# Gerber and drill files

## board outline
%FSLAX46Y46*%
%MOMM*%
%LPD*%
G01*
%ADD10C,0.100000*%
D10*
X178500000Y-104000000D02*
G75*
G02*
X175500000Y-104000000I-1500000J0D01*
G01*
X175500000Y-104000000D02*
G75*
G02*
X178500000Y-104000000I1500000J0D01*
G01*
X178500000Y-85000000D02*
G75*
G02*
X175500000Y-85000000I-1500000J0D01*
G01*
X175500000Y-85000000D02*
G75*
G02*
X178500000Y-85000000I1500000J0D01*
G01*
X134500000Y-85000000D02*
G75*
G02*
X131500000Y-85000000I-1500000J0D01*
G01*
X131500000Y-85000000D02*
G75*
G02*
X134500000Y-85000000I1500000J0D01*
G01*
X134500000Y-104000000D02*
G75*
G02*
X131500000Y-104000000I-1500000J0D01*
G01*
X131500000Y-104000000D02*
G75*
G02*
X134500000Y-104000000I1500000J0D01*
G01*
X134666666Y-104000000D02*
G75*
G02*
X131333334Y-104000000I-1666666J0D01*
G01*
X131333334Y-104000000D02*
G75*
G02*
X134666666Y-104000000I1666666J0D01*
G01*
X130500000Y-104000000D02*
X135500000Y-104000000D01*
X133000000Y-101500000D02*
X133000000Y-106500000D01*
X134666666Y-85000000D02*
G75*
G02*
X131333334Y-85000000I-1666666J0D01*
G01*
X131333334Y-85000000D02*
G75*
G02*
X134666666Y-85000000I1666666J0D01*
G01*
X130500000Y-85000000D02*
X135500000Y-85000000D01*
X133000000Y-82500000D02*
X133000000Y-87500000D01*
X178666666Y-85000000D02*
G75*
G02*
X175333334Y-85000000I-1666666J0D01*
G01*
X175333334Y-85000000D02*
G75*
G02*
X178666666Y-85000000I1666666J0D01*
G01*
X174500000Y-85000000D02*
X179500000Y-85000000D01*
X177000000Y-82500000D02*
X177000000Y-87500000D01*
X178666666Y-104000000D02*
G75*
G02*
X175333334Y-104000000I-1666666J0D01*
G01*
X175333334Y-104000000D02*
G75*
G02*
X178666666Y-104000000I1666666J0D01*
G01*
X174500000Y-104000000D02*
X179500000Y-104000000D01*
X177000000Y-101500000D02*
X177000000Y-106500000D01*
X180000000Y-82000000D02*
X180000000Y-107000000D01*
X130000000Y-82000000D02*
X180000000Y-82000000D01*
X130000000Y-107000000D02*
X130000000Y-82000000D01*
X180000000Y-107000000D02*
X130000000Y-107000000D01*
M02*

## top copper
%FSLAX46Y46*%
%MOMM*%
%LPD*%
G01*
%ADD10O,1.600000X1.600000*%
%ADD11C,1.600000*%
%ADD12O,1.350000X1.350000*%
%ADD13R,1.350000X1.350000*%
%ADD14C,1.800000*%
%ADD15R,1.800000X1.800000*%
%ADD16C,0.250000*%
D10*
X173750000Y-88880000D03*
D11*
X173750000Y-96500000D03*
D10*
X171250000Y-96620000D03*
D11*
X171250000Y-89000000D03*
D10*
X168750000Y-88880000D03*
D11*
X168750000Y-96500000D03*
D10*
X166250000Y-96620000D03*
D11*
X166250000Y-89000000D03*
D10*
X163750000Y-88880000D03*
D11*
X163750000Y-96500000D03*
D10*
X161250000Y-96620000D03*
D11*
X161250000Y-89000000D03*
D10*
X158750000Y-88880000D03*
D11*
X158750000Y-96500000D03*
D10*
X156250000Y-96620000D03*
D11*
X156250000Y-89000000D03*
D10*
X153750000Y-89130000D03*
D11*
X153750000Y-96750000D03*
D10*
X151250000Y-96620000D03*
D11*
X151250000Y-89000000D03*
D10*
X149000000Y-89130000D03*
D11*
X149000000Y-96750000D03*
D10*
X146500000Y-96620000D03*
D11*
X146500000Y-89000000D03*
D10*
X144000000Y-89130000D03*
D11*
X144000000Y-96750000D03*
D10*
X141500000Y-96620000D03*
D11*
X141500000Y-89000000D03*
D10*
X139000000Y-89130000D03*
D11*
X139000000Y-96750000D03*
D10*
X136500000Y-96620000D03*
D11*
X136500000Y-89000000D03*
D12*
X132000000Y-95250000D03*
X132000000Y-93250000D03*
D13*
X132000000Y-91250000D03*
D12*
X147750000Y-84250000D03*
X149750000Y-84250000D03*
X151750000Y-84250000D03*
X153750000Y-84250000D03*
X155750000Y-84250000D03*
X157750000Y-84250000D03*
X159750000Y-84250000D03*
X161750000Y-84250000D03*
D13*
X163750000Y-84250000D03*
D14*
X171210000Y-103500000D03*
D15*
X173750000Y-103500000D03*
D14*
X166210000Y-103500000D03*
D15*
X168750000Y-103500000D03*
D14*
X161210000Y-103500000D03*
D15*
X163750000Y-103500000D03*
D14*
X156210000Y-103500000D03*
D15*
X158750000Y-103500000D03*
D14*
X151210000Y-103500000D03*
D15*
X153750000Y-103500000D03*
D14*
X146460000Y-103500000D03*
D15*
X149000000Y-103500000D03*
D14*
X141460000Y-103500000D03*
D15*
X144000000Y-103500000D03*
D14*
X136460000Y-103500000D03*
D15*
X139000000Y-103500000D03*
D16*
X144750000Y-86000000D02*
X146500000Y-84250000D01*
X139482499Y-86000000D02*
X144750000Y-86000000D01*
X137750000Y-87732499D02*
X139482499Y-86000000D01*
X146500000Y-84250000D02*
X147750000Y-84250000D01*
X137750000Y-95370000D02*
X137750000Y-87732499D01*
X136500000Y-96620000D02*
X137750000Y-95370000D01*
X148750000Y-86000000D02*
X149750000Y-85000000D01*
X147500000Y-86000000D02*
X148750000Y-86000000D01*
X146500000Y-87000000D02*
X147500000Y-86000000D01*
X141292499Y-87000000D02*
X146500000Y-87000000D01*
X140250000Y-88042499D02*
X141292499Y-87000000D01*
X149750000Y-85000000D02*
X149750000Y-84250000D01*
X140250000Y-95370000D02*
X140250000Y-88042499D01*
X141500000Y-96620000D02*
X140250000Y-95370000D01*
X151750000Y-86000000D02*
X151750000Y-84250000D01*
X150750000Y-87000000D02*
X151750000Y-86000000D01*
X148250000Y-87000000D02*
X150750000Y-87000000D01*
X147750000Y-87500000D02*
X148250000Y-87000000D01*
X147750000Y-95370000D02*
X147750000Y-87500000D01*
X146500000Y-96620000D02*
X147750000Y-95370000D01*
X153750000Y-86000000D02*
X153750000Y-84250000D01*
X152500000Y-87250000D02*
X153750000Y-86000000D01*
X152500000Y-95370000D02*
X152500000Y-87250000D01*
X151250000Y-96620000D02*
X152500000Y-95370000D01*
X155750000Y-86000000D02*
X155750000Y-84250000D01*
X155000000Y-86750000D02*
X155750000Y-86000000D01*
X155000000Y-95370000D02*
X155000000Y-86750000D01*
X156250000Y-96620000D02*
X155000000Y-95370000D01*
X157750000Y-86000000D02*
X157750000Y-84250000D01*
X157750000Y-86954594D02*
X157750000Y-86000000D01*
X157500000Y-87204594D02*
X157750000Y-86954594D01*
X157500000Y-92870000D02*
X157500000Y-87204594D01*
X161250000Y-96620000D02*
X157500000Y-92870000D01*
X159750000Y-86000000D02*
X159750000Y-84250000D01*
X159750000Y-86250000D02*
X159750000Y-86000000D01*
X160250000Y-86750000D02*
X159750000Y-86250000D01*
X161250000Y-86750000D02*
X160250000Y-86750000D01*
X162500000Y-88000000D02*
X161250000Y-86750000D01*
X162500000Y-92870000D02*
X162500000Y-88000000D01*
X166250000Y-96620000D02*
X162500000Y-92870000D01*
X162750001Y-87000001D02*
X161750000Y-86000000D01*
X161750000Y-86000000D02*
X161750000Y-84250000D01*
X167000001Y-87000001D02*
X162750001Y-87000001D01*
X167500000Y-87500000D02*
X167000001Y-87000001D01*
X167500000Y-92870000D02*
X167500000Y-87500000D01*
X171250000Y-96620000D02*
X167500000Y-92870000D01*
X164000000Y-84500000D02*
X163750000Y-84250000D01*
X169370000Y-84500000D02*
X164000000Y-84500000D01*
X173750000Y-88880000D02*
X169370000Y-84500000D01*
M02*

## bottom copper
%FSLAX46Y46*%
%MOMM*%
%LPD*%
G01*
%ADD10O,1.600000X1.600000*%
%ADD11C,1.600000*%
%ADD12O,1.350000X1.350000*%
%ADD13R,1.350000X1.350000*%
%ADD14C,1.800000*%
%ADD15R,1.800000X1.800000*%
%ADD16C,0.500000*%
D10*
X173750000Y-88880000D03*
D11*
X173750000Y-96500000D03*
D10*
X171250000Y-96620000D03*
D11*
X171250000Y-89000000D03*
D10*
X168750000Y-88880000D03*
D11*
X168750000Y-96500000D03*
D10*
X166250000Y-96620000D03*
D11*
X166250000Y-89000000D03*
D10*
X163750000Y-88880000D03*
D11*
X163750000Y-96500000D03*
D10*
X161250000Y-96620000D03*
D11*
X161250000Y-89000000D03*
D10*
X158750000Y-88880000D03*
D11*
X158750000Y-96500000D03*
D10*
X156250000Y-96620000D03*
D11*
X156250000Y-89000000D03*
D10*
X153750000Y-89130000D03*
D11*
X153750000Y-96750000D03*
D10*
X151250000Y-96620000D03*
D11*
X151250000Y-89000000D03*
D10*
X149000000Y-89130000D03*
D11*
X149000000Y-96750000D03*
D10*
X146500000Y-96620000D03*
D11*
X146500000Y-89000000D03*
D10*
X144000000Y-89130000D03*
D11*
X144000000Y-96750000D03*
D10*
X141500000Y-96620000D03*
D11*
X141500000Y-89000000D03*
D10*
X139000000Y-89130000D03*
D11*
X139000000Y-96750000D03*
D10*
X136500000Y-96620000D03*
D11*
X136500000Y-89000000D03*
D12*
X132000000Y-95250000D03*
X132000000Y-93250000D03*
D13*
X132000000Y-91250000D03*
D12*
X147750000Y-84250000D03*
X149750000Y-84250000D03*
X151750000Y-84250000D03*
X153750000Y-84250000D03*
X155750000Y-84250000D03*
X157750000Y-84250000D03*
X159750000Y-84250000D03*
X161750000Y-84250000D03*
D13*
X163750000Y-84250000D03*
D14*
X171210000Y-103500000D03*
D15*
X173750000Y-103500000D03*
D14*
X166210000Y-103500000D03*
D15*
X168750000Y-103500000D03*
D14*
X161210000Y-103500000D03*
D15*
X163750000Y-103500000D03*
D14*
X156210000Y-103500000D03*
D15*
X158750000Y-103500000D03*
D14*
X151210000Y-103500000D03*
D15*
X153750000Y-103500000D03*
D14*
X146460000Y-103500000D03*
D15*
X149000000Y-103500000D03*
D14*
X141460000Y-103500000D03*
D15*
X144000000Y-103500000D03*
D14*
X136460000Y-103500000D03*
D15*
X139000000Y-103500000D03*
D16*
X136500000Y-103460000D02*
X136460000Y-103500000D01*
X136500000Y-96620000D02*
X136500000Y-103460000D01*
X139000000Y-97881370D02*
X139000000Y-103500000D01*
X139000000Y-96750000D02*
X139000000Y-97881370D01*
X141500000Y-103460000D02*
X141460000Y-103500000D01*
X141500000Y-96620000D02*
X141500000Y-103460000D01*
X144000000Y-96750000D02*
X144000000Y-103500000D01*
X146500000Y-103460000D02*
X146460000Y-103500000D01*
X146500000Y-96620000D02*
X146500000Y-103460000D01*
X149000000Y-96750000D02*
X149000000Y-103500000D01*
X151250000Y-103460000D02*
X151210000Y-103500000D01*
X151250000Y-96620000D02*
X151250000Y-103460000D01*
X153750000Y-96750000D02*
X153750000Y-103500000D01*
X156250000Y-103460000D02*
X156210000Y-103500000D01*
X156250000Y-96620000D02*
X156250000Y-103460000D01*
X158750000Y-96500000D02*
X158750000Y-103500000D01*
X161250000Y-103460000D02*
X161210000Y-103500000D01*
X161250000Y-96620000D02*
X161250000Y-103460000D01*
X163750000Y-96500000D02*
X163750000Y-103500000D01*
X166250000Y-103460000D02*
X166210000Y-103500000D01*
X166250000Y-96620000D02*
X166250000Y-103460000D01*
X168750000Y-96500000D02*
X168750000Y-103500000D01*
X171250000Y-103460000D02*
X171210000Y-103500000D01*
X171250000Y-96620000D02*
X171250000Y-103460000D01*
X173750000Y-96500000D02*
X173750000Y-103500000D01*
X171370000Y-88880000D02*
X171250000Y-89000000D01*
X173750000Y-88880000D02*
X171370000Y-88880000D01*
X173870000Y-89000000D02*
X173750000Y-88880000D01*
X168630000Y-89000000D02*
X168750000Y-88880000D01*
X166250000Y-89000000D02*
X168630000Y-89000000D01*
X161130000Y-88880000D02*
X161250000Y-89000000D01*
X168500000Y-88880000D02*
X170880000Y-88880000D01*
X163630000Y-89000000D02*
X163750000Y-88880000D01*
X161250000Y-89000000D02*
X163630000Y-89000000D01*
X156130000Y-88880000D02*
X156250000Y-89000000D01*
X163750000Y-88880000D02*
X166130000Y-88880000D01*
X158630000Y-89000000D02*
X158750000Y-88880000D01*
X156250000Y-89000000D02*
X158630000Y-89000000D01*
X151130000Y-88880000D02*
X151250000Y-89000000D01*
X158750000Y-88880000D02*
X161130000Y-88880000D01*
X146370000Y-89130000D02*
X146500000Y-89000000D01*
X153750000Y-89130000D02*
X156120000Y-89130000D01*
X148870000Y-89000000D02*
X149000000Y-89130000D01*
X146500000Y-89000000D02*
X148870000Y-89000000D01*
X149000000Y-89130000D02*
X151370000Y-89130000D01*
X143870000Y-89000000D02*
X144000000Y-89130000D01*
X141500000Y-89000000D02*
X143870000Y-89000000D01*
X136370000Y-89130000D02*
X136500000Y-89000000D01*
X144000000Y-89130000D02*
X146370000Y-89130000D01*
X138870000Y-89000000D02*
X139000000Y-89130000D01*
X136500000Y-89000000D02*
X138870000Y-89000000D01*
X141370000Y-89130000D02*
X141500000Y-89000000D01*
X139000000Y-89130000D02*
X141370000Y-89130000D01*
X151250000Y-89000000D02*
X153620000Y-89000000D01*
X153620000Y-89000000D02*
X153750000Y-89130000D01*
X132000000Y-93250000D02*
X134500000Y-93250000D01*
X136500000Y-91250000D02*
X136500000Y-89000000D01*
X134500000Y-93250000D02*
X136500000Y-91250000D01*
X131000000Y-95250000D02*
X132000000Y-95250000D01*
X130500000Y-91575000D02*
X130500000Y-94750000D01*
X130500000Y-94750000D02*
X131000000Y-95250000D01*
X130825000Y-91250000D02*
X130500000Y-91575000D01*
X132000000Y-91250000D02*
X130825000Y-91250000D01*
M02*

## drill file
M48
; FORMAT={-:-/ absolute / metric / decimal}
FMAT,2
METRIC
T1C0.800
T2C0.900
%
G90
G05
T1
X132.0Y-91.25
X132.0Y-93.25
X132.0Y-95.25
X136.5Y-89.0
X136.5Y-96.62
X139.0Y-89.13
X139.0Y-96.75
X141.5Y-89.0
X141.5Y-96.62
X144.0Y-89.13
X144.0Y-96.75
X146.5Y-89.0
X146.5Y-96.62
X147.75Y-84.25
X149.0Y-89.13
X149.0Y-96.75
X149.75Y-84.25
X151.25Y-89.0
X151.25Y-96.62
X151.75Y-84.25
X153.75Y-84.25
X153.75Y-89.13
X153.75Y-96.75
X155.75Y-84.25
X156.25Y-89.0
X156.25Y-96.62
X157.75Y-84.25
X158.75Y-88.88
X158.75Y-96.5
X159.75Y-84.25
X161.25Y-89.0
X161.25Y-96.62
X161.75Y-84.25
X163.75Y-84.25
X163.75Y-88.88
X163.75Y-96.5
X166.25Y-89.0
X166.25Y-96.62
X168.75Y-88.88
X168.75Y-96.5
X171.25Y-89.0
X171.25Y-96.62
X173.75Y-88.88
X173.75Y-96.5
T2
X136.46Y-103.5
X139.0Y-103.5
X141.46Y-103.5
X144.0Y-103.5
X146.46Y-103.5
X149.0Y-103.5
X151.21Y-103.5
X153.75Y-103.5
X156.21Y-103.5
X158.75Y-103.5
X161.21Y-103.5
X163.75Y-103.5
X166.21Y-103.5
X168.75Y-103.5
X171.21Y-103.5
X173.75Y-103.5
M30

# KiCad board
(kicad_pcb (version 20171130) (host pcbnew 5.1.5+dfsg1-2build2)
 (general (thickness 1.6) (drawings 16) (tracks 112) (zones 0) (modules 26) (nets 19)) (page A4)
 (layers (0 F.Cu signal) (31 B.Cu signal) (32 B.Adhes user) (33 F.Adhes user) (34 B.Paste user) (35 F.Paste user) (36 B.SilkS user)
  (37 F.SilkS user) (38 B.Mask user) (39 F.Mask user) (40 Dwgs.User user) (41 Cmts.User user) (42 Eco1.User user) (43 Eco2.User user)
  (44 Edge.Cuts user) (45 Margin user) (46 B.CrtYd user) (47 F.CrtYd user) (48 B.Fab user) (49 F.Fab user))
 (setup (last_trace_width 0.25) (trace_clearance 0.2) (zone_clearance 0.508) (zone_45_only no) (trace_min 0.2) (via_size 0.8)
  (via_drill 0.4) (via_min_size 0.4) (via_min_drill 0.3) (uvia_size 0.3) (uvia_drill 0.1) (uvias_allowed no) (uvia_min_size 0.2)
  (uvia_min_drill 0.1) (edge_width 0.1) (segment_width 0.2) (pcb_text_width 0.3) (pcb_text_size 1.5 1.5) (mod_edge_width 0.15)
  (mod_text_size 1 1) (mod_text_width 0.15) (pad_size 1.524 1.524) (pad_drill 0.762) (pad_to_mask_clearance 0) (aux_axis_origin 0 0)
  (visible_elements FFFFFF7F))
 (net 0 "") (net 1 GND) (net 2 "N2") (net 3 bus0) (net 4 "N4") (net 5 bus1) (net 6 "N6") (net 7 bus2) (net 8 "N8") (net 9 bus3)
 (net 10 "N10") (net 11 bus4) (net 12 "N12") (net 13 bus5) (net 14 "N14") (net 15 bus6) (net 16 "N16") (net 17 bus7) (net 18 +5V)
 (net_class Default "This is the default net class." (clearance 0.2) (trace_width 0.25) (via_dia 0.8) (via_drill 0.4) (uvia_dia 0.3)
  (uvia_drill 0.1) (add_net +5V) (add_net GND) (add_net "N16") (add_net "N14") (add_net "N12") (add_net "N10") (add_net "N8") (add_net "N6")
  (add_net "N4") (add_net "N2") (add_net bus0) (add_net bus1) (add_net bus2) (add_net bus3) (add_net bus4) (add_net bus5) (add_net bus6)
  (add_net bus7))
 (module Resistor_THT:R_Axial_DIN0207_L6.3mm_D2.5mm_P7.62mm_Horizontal (layer F.Cu) (at 173.75 96.5 90)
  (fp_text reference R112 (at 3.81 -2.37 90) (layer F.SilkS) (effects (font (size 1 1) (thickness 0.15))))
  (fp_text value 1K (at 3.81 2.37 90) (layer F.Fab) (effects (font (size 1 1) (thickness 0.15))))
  (pad 2 thru_hole oval (at 7.62 0 90) (size 1.6 1.6) (drill 0.8) (layers *.Cu *.Mask) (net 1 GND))
  (pad 1 thru_hole circle (at 0 0 90) (size 1.6 1.6) (drill 0.8) (layers *.Cu *.Mask) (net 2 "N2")))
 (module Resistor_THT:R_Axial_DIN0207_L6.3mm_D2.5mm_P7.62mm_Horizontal (layer F.Cu) (at 171.25 89 270)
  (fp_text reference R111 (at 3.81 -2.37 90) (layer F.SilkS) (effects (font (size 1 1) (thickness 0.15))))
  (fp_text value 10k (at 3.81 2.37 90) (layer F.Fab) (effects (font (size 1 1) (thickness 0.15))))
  (pad 2 thru_hole oval (at 7.62 0 270) (size 1.6 1.6) (drill 0.8) (layers *.Cu *.Mask) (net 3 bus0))
  (pad 1 thru_hole circle (at 0 0 270) (size 1.6 1.6) (drill 0.8) (layers *.Cu *.Mask) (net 1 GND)))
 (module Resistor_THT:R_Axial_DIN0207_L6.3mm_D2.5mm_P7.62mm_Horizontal (layer F.Cu) (at 168.75 96.5 90)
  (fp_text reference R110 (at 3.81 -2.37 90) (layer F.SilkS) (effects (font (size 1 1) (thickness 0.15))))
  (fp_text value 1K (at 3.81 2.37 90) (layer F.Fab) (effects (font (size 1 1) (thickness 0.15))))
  (pad 2 thru_hole oval (at 7.62 0 90) (size 1.6 1.6) (drill 0.8) (layers *.Cu *.Mask) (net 1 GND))
  (pad 1 thru_hole circle (at 0 0 90) (size 1.6 1.6) (drill 0.8) (layers *.Cu *.Mask) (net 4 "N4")))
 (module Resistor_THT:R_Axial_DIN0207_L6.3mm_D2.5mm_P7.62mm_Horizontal (layer F.Cu) (at 166.25 89 270)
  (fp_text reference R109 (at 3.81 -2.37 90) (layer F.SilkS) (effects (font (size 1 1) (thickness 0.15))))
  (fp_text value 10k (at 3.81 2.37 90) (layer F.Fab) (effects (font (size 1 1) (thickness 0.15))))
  (pad 2 thru_hole oval (at 7.62 0 270) (size 1.6 1.6) (drill 0.8) (layers *.Cu *.Mask) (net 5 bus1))
  (pad 1 thru_hole circle (at 0 0 270) (size 1.6 1.6) (drill 0.8) (layers *.Cu *.Mask) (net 1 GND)))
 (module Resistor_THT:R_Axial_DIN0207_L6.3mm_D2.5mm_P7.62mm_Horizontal (layer F.Cu) (at 163.75 96.5 90)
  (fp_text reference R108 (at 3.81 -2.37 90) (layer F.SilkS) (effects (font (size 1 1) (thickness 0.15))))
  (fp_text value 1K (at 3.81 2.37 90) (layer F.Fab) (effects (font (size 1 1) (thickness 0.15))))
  (pad 2 thru_hole oval (at 7.62 0 90) (size 1.6 1.6) (drill 0.8) (layers *.Cu *.Mask) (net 1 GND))
  (pad 1 thru_hole circle (at 0 0 90) (size 1.6 1.6) (drill 0.8) (layers *.Cu *.Mask) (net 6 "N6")))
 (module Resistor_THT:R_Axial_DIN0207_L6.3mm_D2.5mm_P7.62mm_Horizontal (layer F.Cu) (at 161.25 89 270)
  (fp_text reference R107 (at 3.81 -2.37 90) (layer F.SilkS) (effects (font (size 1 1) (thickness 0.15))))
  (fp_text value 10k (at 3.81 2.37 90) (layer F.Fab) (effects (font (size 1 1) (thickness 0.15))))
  (pad 2 thru_hole oval (at 7.62 0 270) (size 1.6 1.6) (drill 0.8) (layers *.Cu *.Mask) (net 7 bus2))
  (pad 1 thru_hole circle (at 0 0 270) (size 1.6 1.6) (drill 0.8) (layers *.Cu *.Mask) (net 1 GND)))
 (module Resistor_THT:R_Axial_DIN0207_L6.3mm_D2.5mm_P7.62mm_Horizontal (layer F.Cu) (at 158.75 96.5 90)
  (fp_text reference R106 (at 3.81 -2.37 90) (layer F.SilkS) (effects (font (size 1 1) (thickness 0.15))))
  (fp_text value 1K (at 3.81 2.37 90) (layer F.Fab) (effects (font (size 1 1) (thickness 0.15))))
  (pad 2 thru_hole oval (at 7.62 0 90) (size 1.6 1.6) (drill 0.8) (layers *.Cu *.Mask) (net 1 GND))
  (pad 1 thru_hole circle (at 0 0 90) (size 1.6 1.6) (drill 0.8) (layers *.Cu *.Mask) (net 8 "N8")))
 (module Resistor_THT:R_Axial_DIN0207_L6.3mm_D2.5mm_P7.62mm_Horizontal (layer F.Cu) (at 156.25 89 270)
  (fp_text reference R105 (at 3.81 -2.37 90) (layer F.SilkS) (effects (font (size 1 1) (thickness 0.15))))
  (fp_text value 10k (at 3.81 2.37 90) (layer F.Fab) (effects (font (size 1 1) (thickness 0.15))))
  (pad 2 thru_hole oval (at 7.62 0 270) (size 1.6 1.6) (drill 0.8) (layers *.Cu *.Mask) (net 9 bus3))
  (pad 1 thru_hole circle (at 0 0 270) (size 1.6 1.6) (drill 0.8) (layers *.Cu *.Mask) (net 1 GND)))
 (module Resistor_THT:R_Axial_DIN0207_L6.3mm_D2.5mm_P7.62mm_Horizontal (layer F.Cu) (at 153.75 96.75 90)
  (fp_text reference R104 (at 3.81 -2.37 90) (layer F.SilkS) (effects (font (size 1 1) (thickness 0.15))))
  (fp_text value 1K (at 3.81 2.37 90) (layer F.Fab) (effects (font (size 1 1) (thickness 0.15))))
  (pad 2 thru_hole oval (at 7.62 0 90) (size 1.6 1.6) (drill 0.8) (layers *.Cu *.Mask) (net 1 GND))
  (pad 1 thru_hole circle (at 0 0 90) (size 1.6 1.6) (drill 0.8) (layers *.Cu *.Mask) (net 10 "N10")))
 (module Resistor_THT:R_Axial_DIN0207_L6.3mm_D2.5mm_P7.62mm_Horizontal (layer F.Cu) (at 151.25 89 270)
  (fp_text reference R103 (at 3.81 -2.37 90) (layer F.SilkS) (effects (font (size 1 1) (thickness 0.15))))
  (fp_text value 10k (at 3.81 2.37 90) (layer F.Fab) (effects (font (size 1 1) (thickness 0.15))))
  (pad 2 thru_hole oval (at 7.62 0 270) (size 1.6 1.6) (drill 0.8) (layers *.Cu *.Mask) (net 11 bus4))
  (pad 1 thru_hole circle (at 0 0 270) (size 1.6 1.6) (drill 0.8) (layers *.Cu *.Mask) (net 1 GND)))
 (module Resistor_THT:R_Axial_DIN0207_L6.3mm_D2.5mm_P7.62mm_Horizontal (layer F.Cu) (at 149 96.75 90)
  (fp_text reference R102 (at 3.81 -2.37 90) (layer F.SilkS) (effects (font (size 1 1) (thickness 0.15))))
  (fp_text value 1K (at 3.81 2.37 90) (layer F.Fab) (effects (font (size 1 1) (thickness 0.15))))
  (pad 2 thru_hole oval (at 7.62 0 90) (size 1.6 1.6) (drill 0.8) (layers *.Cu *.Mask) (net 1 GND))
  (pad 1 thru_hole circle (at 0 0 90) (size 1.6 1.6) (drill 0.8) (layers *.Cu *.Mask) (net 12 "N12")))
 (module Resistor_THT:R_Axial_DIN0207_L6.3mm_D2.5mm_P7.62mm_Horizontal (layer F.Cu) (at 146.5 89 270)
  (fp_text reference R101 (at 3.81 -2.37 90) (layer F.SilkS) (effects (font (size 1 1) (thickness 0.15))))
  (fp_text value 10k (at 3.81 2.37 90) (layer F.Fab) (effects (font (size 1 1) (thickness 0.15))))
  (pad 2 thru_hole oval (at 7.62 0 270) (size 1.6 1.6) (drill 0.8) (layers *.Cu *.Mask) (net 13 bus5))
  (pad 1 thru_hole circle (at 0 0 270) (size 1.6 1.6) (drill 0.8) (layers *.Cu *.Mask) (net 1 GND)))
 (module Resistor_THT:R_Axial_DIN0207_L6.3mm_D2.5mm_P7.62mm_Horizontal (layer F.Cu) (at 144 96.75 90)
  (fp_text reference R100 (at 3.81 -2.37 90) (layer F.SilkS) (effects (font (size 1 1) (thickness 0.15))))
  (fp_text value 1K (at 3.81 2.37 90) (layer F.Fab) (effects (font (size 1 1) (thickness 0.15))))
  (pad 2 thru_hole oval (at 7.62 0 90) (size 1.6 1.6) (drill 0.8) (layers *.Cu *.Mask) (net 1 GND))
  (pad 1 thru_hole circle (at 0 0 90) (size 1.6 1.6) (drill 0.8) (layers *.Cu *.Mask) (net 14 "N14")))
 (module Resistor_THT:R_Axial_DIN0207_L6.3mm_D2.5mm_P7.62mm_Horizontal (layer F.Cu) (at 141.5 89 270)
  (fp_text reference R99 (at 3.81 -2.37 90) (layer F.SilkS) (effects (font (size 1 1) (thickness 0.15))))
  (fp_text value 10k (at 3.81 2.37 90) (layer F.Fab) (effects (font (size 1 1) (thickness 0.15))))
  (pad 2 thru_hole oval (at 7.62 0 270) (size 1.6 1.6) (drill 0.8) (layers *.Cu *.Mask) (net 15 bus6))
  (pad 1 thru_hole circle (at 0 0 270) (size 1.6 1.6) (drill 0.8) (layers *.Cu *.Mask) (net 1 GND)))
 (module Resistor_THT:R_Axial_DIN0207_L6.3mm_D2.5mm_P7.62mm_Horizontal (layer F.Cu) (at 139 96.75 90)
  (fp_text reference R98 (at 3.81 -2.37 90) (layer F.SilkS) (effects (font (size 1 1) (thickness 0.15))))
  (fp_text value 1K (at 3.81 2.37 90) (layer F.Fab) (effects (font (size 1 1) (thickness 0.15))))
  (pad 2 thru_hole oval (at 7.62 0 90) (size 1.6 1.6) (drill 0.8) (layers *.Cu *.Mask) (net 1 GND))
  (pad 1 thru_hole circle (at 0 0 90) (size 1.6 1.6) (drill 0.8) (layers *.Cu *.Mask) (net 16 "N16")))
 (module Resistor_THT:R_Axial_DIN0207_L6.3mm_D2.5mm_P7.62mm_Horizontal (layer F.Cu) (at 136.5 89 270)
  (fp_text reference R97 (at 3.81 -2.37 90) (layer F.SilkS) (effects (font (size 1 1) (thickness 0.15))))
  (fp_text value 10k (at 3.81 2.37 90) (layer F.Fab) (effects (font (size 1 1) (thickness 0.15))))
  (pad 2 thru_hole oval (at 7.62 0 270) (size 1.6 1.6) (drill 0.8) (layers *.Cu *.Mask) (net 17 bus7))
  (pad 1 thru_hole circle (at 0 0 270) (size 1.6 1.6) (drill 0.8) (layers *.Cu *.Mask) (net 1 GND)))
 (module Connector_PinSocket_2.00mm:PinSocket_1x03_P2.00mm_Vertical (layer F.Cu) (at 132 91.25)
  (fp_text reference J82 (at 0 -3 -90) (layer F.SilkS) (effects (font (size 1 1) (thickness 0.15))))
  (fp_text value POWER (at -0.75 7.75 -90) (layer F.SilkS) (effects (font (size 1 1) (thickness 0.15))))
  (pad 3 thru_hole oval (at 0 4) (size 1.35 1.35) (drill 0.8) (layers *.Cu *.Mask) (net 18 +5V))
  (pad 2 thru_hole oval (at 0 2) (size 1.35 1.35) (drill 0.8) (layers *.Cu *.Mask) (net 1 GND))
  (pad 1 thru_hole rect (at 0 0) (size 1.35 1.35) (drill 0.8) (layers *.Cu *.Mask) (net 18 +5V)))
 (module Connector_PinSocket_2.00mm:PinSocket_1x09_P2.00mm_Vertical (layer F.Cu) (at 163.75 84.25 270)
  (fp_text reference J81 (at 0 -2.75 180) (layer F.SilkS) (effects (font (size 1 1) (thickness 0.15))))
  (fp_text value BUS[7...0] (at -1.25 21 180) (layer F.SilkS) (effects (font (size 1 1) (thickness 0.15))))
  (pad 9 thru_hole oval (at 0 16 270) (size 1.35 1.35) (drill 0.8) (layers *.Cu *.Mask) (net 17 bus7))
  (pad 8 thru_hole oval (at 0 14 270) (size 1.35 1.35) (drill 0.8) (layers *.Cu *.Mask) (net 15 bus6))
  (pad 7 thru_hole oval (at 0 12 270) (size 1.35 1.35) (drill 0.8) (layers *.Cu *.Mask) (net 13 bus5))
  (pad 6 thru_hole oval (at 0 10 270) (size 1.35 1.35) (drill 0.8) (layers *.Cu *.Mask) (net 11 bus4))
  (pad 5 thru_hole oval (at 0 8 270) (size 1.35 1.35) (drill 0.8) (layers *.Cu *.Mask) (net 9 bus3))
  (pad 4 thru_hole oval (at 0 6 270) (size 1.35 1.35) (drill 0.8) (layers *.Cu *.Mask) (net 7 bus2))
  (pad 3 thru_hole oval (at 0 4 270) (size 1.35 1.35) (drill 0.8) (layers *.Cu *.Mask) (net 5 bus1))
  (pad 2 thru_hole oval (at 0 2 270) (size 1.35 1.35) (drill 0.8) (layers *.Cu *.Mask) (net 3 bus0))
  (pad 1 thru_hole rect (at 0 0 270) (size 1.35 1.35) (drill 0.8) (layers *.Cu *.Mask) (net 1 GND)))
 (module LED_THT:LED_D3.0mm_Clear (layer F.Cu) (at 173.75 103.5 180)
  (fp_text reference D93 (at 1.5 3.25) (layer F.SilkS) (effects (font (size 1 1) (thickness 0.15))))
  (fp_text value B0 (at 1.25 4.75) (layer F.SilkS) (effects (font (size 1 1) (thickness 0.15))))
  (pad 2 thru_hole circle (at 2.54 0 180) (size 1.8 1.8) (drill 0.9) (layers *.Cu *.Mask) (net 3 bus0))
  (pad 1 thru_hole rect (at 0 0 180) (size 1.8 1.8) (drill 0.9) (layers *.Cu *.Mask) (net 2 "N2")))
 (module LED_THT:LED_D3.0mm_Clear (layer F.Cu) (at 168.75 103.5 180)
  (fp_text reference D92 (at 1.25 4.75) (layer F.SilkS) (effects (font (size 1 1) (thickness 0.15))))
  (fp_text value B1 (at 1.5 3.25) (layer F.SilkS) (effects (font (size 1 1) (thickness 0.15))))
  (pad 2 thru_hole circle (at 2.54 0 180) (size 1.8 1.8) (drill 0.9) (layers *.Cu *.Mask) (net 5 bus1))
  (pad 1 thru_hole rect (at 0 0 180) (size 1.8 1.8) (drill 0.9) (layers *.Cu *.Mask) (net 4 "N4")))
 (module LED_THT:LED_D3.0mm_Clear (layer F.Cu) (at 163.75 103.5 180)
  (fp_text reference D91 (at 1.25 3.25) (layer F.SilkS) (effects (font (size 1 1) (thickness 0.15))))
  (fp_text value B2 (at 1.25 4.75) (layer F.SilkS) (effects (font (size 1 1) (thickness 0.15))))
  (pad 2 thru_hole circle (at 2.54 0 180) (size 1.8 1.8) (drill 0.9) (layers *.Cu *.Mask) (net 7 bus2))
  (pad 1 thru_hole rect (at 0 0 180) (size 1.8 1.8) (drill 0.9) (layers *.Cu *.Mask) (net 6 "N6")))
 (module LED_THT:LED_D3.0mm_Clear (layer F.Cu) (at 158.75 103.5 180)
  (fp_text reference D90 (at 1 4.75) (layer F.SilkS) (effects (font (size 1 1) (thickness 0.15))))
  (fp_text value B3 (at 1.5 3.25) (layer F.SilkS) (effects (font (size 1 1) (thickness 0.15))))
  (pad 2 thru_hole circle (at 2.54 0 180) (size 1.8 1.8) (drill 0.9) (layers *.Cu *.Mask) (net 9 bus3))
  (pad 1 thru_hole rect (at 0 0 180) (size 1.8 1.8) (drill 0.9) (layers *.Cu *.Mask) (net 8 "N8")))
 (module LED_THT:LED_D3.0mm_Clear (layer F.Cu) (at 153.75 103.5 180)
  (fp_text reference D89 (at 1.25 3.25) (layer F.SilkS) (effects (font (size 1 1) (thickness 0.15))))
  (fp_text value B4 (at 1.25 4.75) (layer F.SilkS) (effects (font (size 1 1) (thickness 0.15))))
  (pad 2 thru_hole circle (at 2.54 0 180) (size 1.8 1.8) (drill 0.9) (layers *.Cu *.Mask) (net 11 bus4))
  (pad 1 thru_hole rect (at 0 0 180) (size 1.8 1.8) (drill 0.9) (layers *.Cu *.Mask) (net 10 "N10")))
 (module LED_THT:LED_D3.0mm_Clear (layer F.Cu) (at 149 103.5 180)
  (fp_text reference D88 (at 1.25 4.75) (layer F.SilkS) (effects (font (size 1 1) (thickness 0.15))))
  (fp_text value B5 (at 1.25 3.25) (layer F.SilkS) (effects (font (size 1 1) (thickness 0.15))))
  (pad 2 thru_hole circle (at 2.54 0 180) (size 1.8 1.8) (drill 0.9) (layers *.Cu *.Mask) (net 13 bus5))
  (pad 1 thru_hole rect (at 0 0 180) (size 1.8 1.8) (drill 0.9) (layers *.Cu *.Mask) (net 12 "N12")))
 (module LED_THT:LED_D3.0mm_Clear (layer F.Cu) (at 144 103.5 180)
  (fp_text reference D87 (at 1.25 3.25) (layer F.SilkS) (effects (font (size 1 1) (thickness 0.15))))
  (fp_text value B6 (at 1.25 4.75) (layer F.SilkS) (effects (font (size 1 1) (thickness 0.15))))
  (pad 2 thru_hole circle (at 2.54 0 180) (size 1.8 1.8) (drill 0.9) (layers *.Cu *.Mask) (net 15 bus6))
  (pad 1 thru_hole rect (at 0 0 180) (size 1.8 1.8) (drill 0.9) (layers *.Cu *.Mask) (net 14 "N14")))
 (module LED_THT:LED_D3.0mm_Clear (layer F.Cu) (at 139 103.5 180)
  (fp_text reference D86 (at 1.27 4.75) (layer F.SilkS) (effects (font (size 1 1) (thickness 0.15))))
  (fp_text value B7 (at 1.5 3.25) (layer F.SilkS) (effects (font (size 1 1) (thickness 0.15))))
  (pad 2 thru_hole circle (at 2.54 0 180) (size 1.8 1.8) (drill 0.9) (layers *.Cu *.Mask) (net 17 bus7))
  (pad 1 thru_hole rect (at 0 0 180) (size 1.8 1.8) (drill 0.9) (layers *.Cu *.Mask) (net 16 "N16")))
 (gr_circle (center 177 104) (end 178.5 104) (layer Edge.Cuts) (width 0.1))
 (gr_circle (center 177 85) (end 178.5 85) (layer Edge.Cuts) (width 0.1))
 (gr_circle (center 133 85) (end 134.5 85) (layer Edge.Cuts) (width 0.1))
 (gr_circle (center 133 104) (end 134.5 104) (layer Edge.Cuts) (width 0.1))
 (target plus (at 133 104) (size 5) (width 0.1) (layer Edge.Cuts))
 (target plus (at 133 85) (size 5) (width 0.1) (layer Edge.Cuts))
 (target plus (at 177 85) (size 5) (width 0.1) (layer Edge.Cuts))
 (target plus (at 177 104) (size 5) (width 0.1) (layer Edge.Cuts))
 (gr_line (start 180 82) (end 180 107) (layer Edge.Cuts) (width 0.1))
 (gr_line (start 130 82) (end 180 82) (layer Edge.Cuts) (width 0.1))
 (gr_line (start 130 107) (end 130 82) (layer Edge.Cuts) (width 0.1))
 (gr_line (start 180 107) (end 130 107) (layer Edge.Cuts) (width 0.1))
 (segment (start 136.5 103.46) (end 136.46 103.5) (width 0.5) (layer B.Cu) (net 17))
 (segment (start 136.5 96.62) (end 136.5 103.46) (width 0.5) (layer B.Cu) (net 17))
 (segment (start 144.75 86) (end 146.5 84.25) (width 0.25) (layer F.Cu) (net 17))
 (segment (start 139.482499 86) (end 144.75 86) (width 0.25) (layer F.Cu) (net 17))
 (segment (start 137.75 87.732499) (end 139.482499 86) (width 0.25) (layer F.Cu) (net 17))
 (segment (start 146.5 84.25) (end 147.75 84.25) (width 0.25) (layer F.Cu) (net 17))
 (segment (start 137.75 95.37) (end 137.75 87.732499) (width 0.25) (layer F.Cu) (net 17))
 (segment (start 136.5 96.62) (end 137.75 95.37) (width 0.25) (layer F.Cu) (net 17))
 (segment (start 139 97.88137) (end 139 103.5) (width 0.5) (layer B.Cu) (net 16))
 (segment (start 139 96.75) (end 139 97.88137) (width 0.5) (layer B.Cu) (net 16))
 (segment (start 141.5 103.46) (end 141.46 103.5) (width 0.5) (layer B.Cu) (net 15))
 (segment (start 141.5 96.62) (end 141.5 103.46) (width 0.5) (layer B.Cu) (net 15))
 (segment (start 148.75 86) (end 149.75 85) (width 0.25) (layer F.Cu) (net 15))
 (segment (start 147.5 86) (end 148.75 86) (width 0.25) (layer F.Cu) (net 15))
 (segment (start 146.5 87) (end 147.5 86) (width 0.25) (layer F.Cu) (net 15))
 (segment (start 141.292499 87) (end 146.5 87) (width 0.25) (layer F.Cu) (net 15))
 (segment (start 140.25 88.042499) (end 141.292499 87) (width 0.25) (layer F.Cu) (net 15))
 (segment (start 149.75 85) (end 149.75 84.25) (width 0.25) (layer F.Cu) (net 15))
 (segment (start 140.25 95.37) (end 140.25 88.042499) (width 0.25) (layer F.Cu) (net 15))
 (segment (start 141.5 96.62) (end 140.25 95.37) (width 0.25) (layer F.Cu) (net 15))
 (segment (start 144 96.75) (end 144 103.5) (width 0.5) (layer B.Cu) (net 14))
 (segment (start 146.5 103.46) (end 146.46 103.5) (width 0.5) (layer B.Cu) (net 13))
 (segment (start 146.5 96.62) (end 146.5 103.46) (width 0.5) (layer B.Cu) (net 13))
 (segment (start 151.75 86) (end 151.75 84.25) (width 0.25) (layer F.Cu) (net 13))
 (segment (start 150.75 87) (end 151.75 86) (width 0.25) (layer F.Cu) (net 13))
 (segment (start 148.25 87) (end 150.75 87) (width 0.25) (layer F.Cu) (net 13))
 (segment (start 147.75 87.5) (end 148.25 87) (width 0.25) (layer F.Cu) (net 13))
 (segment (start 147.75 95.37) (end 147.75 87.5) (width 0.25) (layer F.Cu) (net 13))
 (segment (start 146.5 96.62) (end 147.75 95.37) (width 0.25) (layer F.Cu) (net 13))
 (segment (start 149 96.75) (end 149 103.5) (width 0.5) (layer B.Cu) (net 12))
 (segment (start 151.25 103.46) (end 151.21 103.5) (width 0.5) (layer B.Cu) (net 11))
 (segment (start 151.25 96.62) (end 151.25 103.46) (width 0.5) (layer B.Cu) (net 11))
 (segment (start 153.75 86) (end 153.75 84.25) (width 0.25) (layer F.Cu) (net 11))
 (segment (start 152.5 87.25) (end 153.75 86) (width 0.25) (layer F.Cu) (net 11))
 (segment (start 152.5 95.37) (end 152.5 87.25) (width 0.25) (layer F.Cu) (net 11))
 (segment (start 151.25 96.62) (end 152.5 95.37) (width 0.25) (layer F.Cu) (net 11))
 (segment (start 153.75 96.75) (end 153.75 103.5) (width 0.5) (layer B.Cu) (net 10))
 (segment (start 156.25 103.46) (end 156.21 103.5) (width 0.5) (layer B.Cu) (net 9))
 (segment (start 156.25 96.62) (end 156.25 103.46) (width 0.5) (layer B.Cu) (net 9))
 (segment (start 155.75 86) (end 155.75 84.25) (width 0.25) (layer F.Cu) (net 9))
 (segment (start 155 86.75) (end 155.75 86) (width 0.25) (layer F.Cu) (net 9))
 (segment (start 155 95.37) (end 155 86.75) (width 0.25) (layer F.Cu) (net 9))
 (segment (start 156.25 96.62) (end 155 95.37) (width 0.25) (layer F.Cu) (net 9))
 (segment (start 158.75 96.5) (end 158.75 103.5) (width 0.5) (layer B.Cu) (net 8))
 (segment (start 161.25 103.46) (end 161.21 103.5) (width 0.5) (layer B.Cu) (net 7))
 (segment (start 161.25 96.62) (end 161.25 103.46) (width 0.5) (layer B.Cu) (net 7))
 (segment (start 157.75 86) (end 157.75 84.25) (width 0.25) (layer F.Cu) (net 7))
 (segment (start 157.75 86.954594) (end 157.75 86) (width 0.25) (layer F.Cu) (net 7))
 (segment (start 157.5 87.204594) (end 157.75 86.954594) (width 0.25) (layer F.Cu) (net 7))
 (segment (start 157.5 92.87) (end 157.5 87.204594) (width 0.25) (layer F.Cu) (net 7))
 (segment (start 161.25 96.62) (end 157.5 92.87) (width 0.25) (layer F.Cu) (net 7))
 (segment (start 163.75 96.5) (end 163.75 103.5) (width 0.5) (layer B.Cu) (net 6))
 (segment (start 166.25 103.46) (end 166.21 103.5) (width 0.5) (layer B.Cu) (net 5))
 (segment (start 166.25 96.62) (end 166.25 103.46) (width 0.5) (layer B.Cu) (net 5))
 (segment (start 159.75 86) (end 159.75 84.25) (width 0.25) (layer F.Cu) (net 5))
 (segment (start 159.75 86.25) (end 159.75 86) (width 0.25) (layer F.Cu) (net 5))
 (segment (start 160.25 86.75) (end 159.75 86.25) (width 0.25) (layer F.Cu) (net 5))
 (segment (start 161.25 86.75) (end 160.25 86.75) (width 0.25) (layer F.Cu) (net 5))
 (segment (start 162.5 88) (end 161.25 86.75) (width 0.25) (layer F.Cu) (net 5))
 (segment (start 162.5 92.87) (end 162.5 88) (width 0.25) (layer F.Cu) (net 5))
 (segment (start 166.25 96.62) (end 162.5 92.87) (width 0.25) (layer F.Cu) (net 5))
 (segment (start 168.75 96.5) (end 168.75 103.5) (width 0.5) (layer B.Cu) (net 4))
 (segment (start 171.25 103.46) (end 171.21 103.5) (width 0.5) (layer B.Cu) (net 3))
 (segment (start 171.25 96.62) (end 171.25 103.46) (width 0.5) (layer B.Cu) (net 3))
 (segment (start 162.750001 87.000001) (end 161.75 86) (width 0.25) (layer F.Cu) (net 3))
 (segment (start 161.75 86) (end 161.75 84.25) (width 0.25) (layer F.Cu) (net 3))
 (segment (start 167.000001 87.000001) (end 162.750001 87.000001) (width 0.25) (layer F.Cu) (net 3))
 (segment (start 167.5 87.5) (end 167.000001 87.000001) (width 0.25) (layer F.Cu) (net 3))
 (segment (start 167.5 92.87) (end 167.5 87.5) (width 0.25) (layer F.Cu) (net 3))
 (segment (start 171.25 96.62) (end 167.5 92.87) (width 0.25) (layer F.Cu) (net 3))
 (segment (start 173.75 96.5) (end 173.75 103.5) (width 0.5) (layer B.Cu) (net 2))
 (segment (start 171.37 88.88) (end 171.25 89) (width 0.5) (layer B.Cu) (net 1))
 (segment (start 173.75 88.88) (end 171.37 88.88) (width 0.5) (layer B.Cu) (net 1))
 (segment (start 173.87 89) (end 173.75 88.88) (width 0.5) (layer B.Cu) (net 1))
 (segment (start 168.63 89) (end 168.75 88.88) (width 0.5) (layer B.Cu) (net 1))
 (segment (start 166.25 89) (end 168.63 89) (width 0.5) (layer B.Cu) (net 1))
 (segment (start 161.13 88.88) (end 161.25 89) (width 0.5) (layer B.Cu) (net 1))
 (segment (start 168.5 88.88) (end 170.88 88.88) (width 0.5) (layer B.Cu) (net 1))
 (segment (start 163.63 89) (end 163.75 88.88) (width 0.5) (layer B.Cu) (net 1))
 (segment (start 161.25 89) (end 163.63 89) (width 0.5) (layer B.Cu) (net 1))
 (segment (start 156.13 88.88) (end 156.25 89) (width 0.5) (layer B.Cu) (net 1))
 (segment (start 163.75 88.88) (end 166.13 88.88) (width 0.5) (layer B.Cu) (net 1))
 (segment (start 158.63 89) (end 158.75 88.88) (width 0.5) (layer B.Cu) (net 1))
 (segment (start 156.25 89) (end 158.63 89) (width 0.5) (layer B.Cu) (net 1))
 (segment (start 151.13 88.88) (end 151.25 89) (width 0.5) (layer B.Cu) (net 1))
 (segment (start 158.75 88.88) (end 161.13 88.88) (width 0.5) (layer B.Cu) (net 1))
 (segment (start 146.37 89.13) (end 146.5 89) (width 0.5) (layer B.Cu) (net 1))
 (segment (start 153.75 89.13) (end 156.12 89.13) (width 0.5) (layer B.Cu) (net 1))
 (segment (start 148.87 89) (end 149 89.13) (width 0.5) (layer B.Cu) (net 1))
 (segment (start 146.5 89) (end 148.87 89) (width 0.5) (layer B.Cu) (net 1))
 (segment (start 149 89.13) (end 151.37 89.13) (width 0.5) (layer B.Cu) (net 1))
 (segment (start 143.87 89) (end 144 89.13) (width 0.5) (layer B.Cu) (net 1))
 (segment (start 141.5 89) (end 143.87 89) (width 0.5) (layer B.Cu) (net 1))
 (segment (start 136.37 89.13) (end 136.5 89) (width 0.5) (layer B.Cu) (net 1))
 (segment (start 144 89.13) (end 146.37 89.13) (width 0.5) (layer B.Cu) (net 1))
 (segment (start 138.87 89) (end 139 89.13) (width 0.5) (layer B.Cu) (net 1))
 (segment (start 136.5 89) (end 138.87 89) (width 0.5) (layer B.Cu) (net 1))
 (segment (start 141.37 89.13) (end 141.5 89) (width 0.5) (layer B.Cu) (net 1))
 (segment (start 139 89.13) (end 141.37 89.13) (width 0.5) (layer B.Cu) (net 1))
 (segment (start 151.25 89) (end 153.62 89) (width 0.5) (layer B.Cu) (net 1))
 (segment (start 153.62 89) (end 153.75 89.13) (width 0.5) (layer B.Cu) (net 1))
 (segment (start 132 93.25) (end 134.5 93.25) (width 0.5) (layer B.Cu) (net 1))
 (segment (start 136.5 91.25) (end 136.5 89) (width 0.5) (layer B.Cu) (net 1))
 (segment (start 134.5 93.25) (end 136.5 91.25) (width 0.5) (layer B.Cu) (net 1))
 (segment (start 164 84.5) (end 163.75 84.25) (width 0.25) (layer F.Cu) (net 1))
 (segment (start 169.37 84.5) (end 164 84.5) (width 0.25) (layer F.Cu) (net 1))
 (segment (start 173.75 88.88) (end 169.37 84.5) (width 0.25) (layer F.Cu) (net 1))
 (segment (start 131 95.25) (end 132 95.25) (width 0.5) (layer B.Cu) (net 18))
 (segment (start 130.5 91.575) (end 130.5 94.75) (width 0.5) (layer B.Cu) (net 18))
 (segment (start 130.5 94.75) (end 131 95.25) (width 0.5) (layer B.Cu) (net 18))
 (segment (start 130.825 91.25) (end 130.5 91.575) (width 0.5) (layer B.Cu) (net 18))
 (segment (start 132 91.25) (end 130.825 91.25) (width 0.5) (layer B.Cu) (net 18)))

